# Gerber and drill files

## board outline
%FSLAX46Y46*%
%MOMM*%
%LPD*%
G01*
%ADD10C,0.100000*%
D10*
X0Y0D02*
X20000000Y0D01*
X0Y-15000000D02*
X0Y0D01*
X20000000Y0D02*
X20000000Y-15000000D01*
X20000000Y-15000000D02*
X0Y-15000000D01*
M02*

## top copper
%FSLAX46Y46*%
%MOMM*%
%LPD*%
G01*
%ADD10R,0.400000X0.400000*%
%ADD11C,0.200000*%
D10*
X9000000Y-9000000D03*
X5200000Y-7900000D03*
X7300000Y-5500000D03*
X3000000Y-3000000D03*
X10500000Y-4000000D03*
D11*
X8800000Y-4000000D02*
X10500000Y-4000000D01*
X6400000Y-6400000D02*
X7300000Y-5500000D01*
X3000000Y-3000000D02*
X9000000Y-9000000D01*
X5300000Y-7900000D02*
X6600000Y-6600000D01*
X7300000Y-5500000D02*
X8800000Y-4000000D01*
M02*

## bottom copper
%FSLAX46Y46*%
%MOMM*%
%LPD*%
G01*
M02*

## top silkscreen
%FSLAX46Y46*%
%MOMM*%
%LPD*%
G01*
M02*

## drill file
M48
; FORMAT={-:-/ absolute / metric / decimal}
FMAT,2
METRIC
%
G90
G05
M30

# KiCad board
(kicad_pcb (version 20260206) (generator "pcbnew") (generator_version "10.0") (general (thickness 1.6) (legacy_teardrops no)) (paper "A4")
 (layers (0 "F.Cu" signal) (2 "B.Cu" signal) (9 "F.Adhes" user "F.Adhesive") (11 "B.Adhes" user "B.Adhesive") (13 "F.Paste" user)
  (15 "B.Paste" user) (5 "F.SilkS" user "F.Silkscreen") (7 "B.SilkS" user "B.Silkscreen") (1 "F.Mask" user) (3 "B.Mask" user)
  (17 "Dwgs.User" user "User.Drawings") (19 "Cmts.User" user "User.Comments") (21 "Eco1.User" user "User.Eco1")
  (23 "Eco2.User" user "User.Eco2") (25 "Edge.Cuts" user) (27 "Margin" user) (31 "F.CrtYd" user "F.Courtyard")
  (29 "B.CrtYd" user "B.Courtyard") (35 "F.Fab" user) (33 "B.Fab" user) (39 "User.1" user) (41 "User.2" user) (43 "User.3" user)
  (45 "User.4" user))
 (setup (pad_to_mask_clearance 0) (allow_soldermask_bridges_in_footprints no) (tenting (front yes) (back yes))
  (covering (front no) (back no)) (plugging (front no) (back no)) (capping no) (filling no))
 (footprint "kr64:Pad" (layer "F.Cu") (at 9 9)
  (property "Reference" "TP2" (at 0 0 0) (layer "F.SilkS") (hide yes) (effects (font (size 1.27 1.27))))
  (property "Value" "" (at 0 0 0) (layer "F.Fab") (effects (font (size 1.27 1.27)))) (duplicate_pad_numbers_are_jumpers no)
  (pad "1" smd rect (at 0 0) (size 0.4 0.4) (layers "F.Cu" "F.Mask" "F.Paste") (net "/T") (thermal_bridge_angle 45)))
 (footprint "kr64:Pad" (layer "F.Cu") (at 5.2 7.9)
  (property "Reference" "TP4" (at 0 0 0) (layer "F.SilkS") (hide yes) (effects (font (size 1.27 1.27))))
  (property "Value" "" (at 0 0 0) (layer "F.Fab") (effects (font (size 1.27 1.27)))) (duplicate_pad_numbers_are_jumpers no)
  (pad "1" smd rect (at 0 0) (size 0.4 0.4) (layers "F.Cu" "F.Mask" "F.Paste") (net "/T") (thermal_bridge_angle 45)))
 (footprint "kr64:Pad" (layer "F.Cu") (at 7.3 5.5)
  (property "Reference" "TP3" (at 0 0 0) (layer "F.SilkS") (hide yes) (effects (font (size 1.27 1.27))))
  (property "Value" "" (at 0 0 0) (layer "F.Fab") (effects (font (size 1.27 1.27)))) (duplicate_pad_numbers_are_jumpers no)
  (pad "1" smd rect (at 0 0) (size 0.4 0.4) (layers "F.Cu" "F.Mask" "F.Paste") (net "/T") (thermal_bridge_angle 45)))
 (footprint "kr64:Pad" (layer "F.Cu") (at 3 3)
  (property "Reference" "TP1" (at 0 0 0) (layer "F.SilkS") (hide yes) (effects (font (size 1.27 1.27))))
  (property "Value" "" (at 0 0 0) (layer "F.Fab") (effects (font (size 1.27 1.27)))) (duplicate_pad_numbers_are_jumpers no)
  (pad "1" smd rect (at 0 0) (size 0.4 0.4) (layers "F.Cu" "F.Mask" "F.Paste") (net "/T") (thermal_bridge_angle 45)))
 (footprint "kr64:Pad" (layer "F.Cu") (at 10.5 4)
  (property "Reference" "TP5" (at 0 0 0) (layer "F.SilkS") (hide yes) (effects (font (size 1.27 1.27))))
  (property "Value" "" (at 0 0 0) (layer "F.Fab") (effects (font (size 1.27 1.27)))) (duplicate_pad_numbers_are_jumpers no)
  (pad "1" smd rect (at 0 0) (size 0.4 0.4) (layers "F.Cu" "F.Mask" "F.Paste") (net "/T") (thermal_bridge_angle 45)))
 (gr_line (start 0 0) (end 20 0) (stroke (width 0.1) (type default)) (layer "Edge.Cuts"))
 (gr_line (start 0 15) (end 0 0) (stroke (width 0.1) (type default)) (layer "Edge.Cuts"))
 (gr_line (start 20 0) (end 20 15) (stroke (width 0.1) (type default)) (layer "Edge.Cuts"))
 (gr_line (start 20 15) (end 0 15) (stroke (width 0.1) (type default)) (layer "Edge.Cuts"))
 (segment (start 8.8 4) (end 10.5 4) (width 0.2) (layer "F.Cu") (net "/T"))
 (segment (start 6.4 6.4) (end 7.3 5.5) (width 0.2) (layer "F.Cu") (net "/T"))
 (segment (start 3 3) (end 9 9) (width 0.2) (layer "F.Cu") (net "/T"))
 (segment (start 5.3 7.9) (end 6.6 6.6) (width 0.2) (layer "F.Cu") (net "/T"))
 (segment (start 7.3 5.5) (end 8.8 4) (width 0.2) (layer "F.Cu") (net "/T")))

